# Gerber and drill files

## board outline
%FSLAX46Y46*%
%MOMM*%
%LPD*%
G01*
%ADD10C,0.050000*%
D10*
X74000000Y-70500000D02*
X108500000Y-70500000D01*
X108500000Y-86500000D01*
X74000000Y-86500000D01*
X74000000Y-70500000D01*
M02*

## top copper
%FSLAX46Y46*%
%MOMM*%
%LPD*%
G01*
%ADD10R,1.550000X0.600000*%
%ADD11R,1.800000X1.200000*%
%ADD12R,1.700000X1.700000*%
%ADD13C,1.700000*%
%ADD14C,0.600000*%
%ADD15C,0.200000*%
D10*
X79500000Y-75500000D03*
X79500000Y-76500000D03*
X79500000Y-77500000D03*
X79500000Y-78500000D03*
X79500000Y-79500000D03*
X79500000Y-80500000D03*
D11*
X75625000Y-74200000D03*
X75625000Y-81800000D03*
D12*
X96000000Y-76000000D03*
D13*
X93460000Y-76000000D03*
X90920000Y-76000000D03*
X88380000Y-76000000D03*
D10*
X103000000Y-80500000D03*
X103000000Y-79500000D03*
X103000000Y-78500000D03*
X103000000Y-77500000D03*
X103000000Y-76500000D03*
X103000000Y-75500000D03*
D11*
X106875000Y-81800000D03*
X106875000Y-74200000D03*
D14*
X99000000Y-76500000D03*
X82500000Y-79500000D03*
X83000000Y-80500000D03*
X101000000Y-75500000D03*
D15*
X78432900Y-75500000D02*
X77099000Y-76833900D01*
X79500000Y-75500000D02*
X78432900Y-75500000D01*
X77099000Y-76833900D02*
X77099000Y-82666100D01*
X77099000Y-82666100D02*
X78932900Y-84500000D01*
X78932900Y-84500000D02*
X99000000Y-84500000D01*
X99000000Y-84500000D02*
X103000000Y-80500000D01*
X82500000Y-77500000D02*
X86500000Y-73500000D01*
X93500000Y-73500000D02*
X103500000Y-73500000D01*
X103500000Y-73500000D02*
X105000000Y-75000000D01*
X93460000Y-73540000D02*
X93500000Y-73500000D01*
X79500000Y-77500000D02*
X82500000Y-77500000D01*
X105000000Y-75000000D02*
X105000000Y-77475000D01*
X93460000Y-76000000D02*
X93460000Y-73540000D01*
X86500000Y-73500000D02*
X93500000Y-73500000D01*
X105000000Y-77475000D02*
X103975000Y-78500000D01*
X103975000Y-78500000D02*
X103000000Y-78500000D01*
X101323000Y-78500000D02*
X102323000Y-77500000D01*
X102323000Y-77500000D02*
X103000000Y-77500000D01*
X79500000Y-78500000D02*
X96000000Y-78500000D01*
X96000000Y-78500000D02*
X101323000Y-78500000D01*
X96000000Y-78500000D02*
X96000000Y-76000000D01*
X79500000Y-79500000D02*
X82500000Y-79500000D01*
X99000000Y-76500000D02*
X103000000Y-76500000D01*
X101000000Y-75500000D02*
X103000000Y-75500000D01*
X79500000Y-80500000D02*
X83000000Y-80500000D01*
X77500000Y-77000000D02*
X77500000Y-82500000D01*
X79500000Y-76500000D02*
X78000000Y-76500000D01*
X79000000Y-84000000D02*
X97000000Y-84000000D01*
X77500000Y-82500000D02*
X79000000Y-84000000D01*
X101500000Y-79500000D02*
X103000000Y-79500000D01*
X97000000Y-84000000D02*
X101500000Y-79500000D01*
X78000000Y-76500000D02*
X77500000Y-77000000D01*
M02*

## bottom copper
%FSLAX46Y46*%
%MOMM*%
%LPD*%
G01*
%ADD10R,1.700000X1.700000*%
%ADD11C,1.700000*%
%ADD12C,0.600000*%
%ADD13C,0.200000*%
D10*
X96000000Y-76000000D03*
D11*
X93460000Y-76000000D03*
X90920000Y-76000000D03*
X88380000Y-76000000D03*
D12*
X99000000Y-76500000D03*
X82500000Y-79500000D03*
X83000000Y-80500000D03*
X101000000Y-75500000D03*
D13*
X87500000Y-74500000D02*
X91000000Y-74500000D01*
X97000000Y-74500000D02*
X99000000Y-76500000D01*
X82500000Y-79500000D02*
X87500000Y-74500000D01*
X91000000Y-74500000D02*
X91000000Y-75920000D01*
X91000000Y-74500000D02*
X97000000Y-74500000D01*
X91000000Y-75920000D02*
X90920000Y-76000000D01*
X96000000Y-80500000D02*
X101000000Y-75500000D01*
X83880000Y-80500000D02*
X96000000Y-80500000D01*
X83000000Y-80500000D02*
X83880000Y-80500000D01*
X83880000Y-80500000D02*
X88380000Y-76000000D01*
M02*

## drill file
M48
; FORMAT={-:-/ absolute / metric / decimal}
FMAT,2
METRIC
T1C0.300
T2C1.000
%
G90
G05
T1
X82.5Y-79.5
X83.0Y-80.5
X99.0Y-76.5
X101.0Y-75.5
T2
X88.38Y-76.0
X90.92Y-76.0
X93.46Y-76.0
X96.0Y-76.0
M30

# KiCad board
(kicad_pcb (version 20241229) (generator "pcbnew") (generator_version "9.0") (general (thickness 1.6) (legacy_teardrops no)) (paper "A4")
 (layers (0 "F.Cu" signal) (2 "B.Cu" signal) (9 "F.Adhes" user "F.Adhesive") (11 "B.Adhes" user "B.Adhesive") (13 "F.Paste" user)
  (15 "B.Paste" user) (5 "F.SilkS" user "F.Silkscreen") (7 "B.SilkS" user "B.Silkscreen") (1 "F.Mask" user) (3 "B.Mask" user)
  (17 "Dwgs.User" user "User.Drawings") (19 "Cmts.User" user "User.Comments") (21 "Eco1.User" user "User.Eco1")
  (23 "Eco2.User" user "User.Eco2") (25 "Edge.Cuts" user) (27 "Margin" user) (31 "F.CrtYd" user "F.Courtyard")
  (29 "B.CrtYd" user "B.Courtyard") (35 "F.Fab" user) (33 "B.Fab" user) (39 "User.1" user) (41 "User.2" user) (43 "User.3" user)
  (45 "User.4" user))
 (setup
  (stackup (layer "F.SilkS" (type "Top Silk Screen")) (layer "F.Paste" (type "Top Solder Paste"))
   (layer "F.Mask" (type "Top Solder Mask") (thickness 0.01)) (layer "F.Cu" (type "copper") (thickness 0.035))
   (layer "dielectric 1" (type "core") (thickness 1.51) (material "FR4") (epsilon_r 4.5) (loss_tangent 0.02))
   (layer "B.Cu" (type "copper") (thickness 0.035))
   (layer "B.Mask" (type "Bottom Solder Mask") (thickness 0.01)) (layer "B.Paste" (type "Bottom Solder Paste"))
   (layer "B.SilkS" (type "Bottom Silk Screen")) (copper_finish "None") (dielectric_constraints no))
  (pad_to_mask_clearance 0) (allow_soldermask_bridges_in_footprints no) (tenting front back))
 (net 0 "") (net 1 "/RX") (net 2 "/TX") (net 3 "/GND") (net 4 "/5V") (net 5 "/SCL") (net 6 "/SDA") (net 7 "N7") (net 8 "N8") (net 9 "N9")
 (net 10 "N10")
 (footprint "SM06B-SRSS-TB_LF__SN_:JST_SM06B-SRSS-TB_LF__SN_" (layer "F.Cu") (at 79.5 78 -90)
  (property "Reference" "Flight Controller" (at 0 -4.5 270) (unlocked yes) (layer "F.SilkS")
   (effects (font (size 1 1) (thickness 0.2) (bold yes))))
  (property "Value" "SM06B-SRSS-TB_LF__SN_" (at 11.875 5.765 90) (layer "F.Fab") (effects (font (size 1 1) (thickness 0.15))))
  (pad "1" smd rect (at -2.5 0 270) (size 0.6 1.55) (layers "F.Cu" "F.Mask" "F.Paste") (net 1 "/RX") (solder_mask_margin 0.102))
  (pad "2" smd rect (at -1.5 0 270) (size 0.6 1.55) (layers "F.Cu" "F.Mask" "F.Paste") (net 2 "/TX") (solder_mask_margin 0.102))
  (pad "3" smd rect (at -0.5 0 270) (size 0.6 1.55) (layers "F.Cu" "F.Mask" "F.Paste") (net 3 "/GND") (solder_mask_margin 0.102))
  (pad "4" smd rect (at 0.5 0 270) (size 0.6 1.55) (layers "F.Cu" "F.Mask" "F.Paste") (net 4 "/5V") (solder_mask_margin 0.102))
  (pad "5" smd rect (at 1.5 0 270) (size 0.6 1.55) (layers "F.Cu" "F.Mask" "F.Paste") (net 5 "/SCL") (solder_mask_margin 0.102))
  (pad "6" smd rect (at 2.5 0 270) (size 0.6 1.55) (layers "F.Cu" "F.Mask" "F.Paste") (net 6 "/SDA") (solder_mask_margin 0.102))
  (pad "S1" smd rect (at -3.8 3.875 270) (size 1.2 1.8) (layers "F.Cu" "F.Mask" "F.Paste") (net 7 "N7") (solder_mask_margin 0.102))
  (pad "S2" smd rect (at 3.8 3.875 270) (size 1.2 1.8) (layers "F.Cu" "F.Mask" "F.Paste") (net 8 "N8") (solder_mask_margin 0.102)))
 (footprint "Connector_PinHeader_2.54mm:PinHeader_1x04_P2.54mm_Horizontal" (layer "F.Cu") (at 96 76 -90)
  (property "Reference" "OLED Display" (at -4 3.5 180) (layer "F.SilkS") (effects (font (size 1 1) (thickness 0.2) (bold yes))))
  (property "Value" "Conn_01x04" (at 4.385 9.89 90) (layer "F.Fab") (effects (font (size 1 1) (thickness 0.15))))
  (pad "1" thru_hole rect (at 0 0 270) (size 1.7 1.7) (drill 1) (layers "*.Cu" "*.Mask") (remove_unused_layers no) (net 4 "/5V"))
  (pad "2" thru_hole circle (at 0 2.54 270) (size 1.7 1.7) (drill 1) (layers "*.Cu" "*.Mask") (remove_unused_layers no) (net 3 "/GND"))
  (pad "3" thru_hole circle (at 0 5.08 270) (size 1.7 1.7) (drill 1) (layers "*.Cu" "*.Mask") (remove_unused_layers no) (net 5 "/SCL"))
  (pad "4" thru_hole circle (at 0 7.62 270) (size 1.7 1.7) (drill 1) (layers "*.Cu" "*.Mask") (remove_unused_layers no) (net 6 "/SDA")))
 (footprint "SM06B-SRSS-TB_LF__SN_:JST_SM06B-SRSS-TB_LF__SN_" (layer "F.Cu") (at 103 78 90)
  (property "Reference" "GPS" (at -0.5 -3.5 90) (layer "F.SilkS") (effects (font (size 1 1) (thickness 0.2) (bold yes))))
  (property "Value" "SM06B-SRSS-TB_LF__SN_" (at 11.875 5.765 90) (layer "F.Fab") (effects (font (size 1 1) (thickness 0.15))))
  (pad "1" smd rect (at -2.5 0 90) (size 0.6 1.55) (layers "F.Cu" "F.Mask" "F.Paste") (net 1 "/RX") (solder_mask_margin 0.102))
  (pad "2" smd rect (at -1.5 0 90) (size 0.6 1.55) (layers "F.Cu" "F.Mask" "F.Paste") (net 2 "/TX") (solder_mask_margin 0.102))
  (pad "3" smd rect (at -0.5 0 90) (size 0.6 1.55) (layers "F.Cu" "F.Mask" "F.Paste") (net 3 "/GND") (solder_mask_margin 0.102))
  (pad "4" smd rect (at 0.5 0 90) (size 0.6 1.55) (layers "F.Cu" "F.Mask" "F.Paste") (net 4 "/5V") (solder_mask_margin 0.102))
  (pad "5" smd rect (at 1.5 0 90) (size 0.6 1.55) (layers "F.Cu" "F.Mask" "F.Paste") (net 5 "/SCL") (solder_mask_margin 0.102))
  (pad "6" smd rect (at 2.5 0 90) (size 0.6 1.55) (layers "F.Cu" "F.Mask" "F.Paste") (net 6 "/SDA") (solder_mask_margin 0.102))
  (pad "S1" smd rect (at -3.8 3.875 90) (size 1.2 1.8) (layers "F.Cu" "F.Mask" "F.Paste") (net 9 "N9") (solder_mask_margin 0.102))
  (pad "S2" smd rect (at 3.8 3.875 90) (size 1.2 1.8) (layers "F.Cu" "F.Mask" "F.Paste") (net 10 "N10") (solder_mask_margin 0.102)))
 (gr_rect (start 74 70.5) (end 108.5 86.5) (stroke (width 0.05) (type default)) (fill no) (layer "Edge.Cuts"))
 (segment (start 78.4329 75.5) (end 77.099 76.8339) (width 0.2) (layer "F.Cu") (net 1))
 (segment (start 79.5 75.5) (end 78.4329 75.5) (width 0.2) (layer "F.Cu") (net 1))
 (segment (start 77.099 76.8339) (end 77.099 82.6661) (width 0.2) (layer "F.Cu") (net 1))
 (segment (start 77.099 82.6661) (end 78.9329 84.5) (width 0.2) (layer "F.Cu") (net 1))
 (segment (start 78.9329 84.5) (end 99 84.5) (width 0.2) (layer "F.Cu") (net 1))
 (segment (start 99 84.5) (end 103 80.5) (width 0.2) (layer "F.Cu") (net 1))
 (segment (start 82.5 77.5) (end 86.5 73.5) (width 0.2) (layer "F.Cu") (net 3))
 (segment (start 93.5 73.5) (end 103.5 73.5) (width 0.2) (layer "F.Cu") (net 3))
 (segment (start 103.5 73.5) (end 105 75) (width 0.2) (layer "F.Cu") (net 3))
 (segment (start 93.46 73.54) (end 93.5 73.5) (width 0.2) (layer "F.Cu") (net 3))
 (segment (start 79.5 77.5) (end 82.5 77.5) (width 0.2) (layer "F.Cu") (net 3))
 (segment (start 105 75) (end 105 77.475) (width 0.2) (layer "F.Cu") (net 3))
 (segment (start 93.46 76) (end 93.46 73.54) (width 0.2) (layer "F.Cu") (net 3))
 (segment (start 86.5 73.5) (end 93.5 73.5) (width 0.2) (layer "F.Cu") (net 3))
 (segment (start 105 77.475) (end 103.975 78.5) (width 0.2) (layer "F.Cu") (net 3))
 (segment (start 103.975 78.5) (end 103 78.5) (width 0.2) (layer "F.Cu") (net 3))
 (segment (start 101.323 78.5) (end 102.323 77.5) (width 0.2) (layer "F.Cu") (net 4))
 (segment (start 102.323 77.5) (end 103 77.5) (width 0.2) (layer "F.Cu") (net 4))
 (segment (start 79.5 78.5) (end 96 78.5) (width 0.2) (layer "F.Cu") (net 4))
 (segment (start 96 78.5) (end 101.323 78.5) (width 0.2) (layer "F.Cu") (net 4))
 (segment (start 96 78.5) (end 96 76) (width 0.2) (layer "F.Cu") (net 4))
 (segment (start 79.5 79.5) (end 82.5 79.5) (width 0.2) (layer "F.Cu") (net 5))
 (segment (start 99 76.5) (end 103 76.5) (width 0.2) (layer "F.Cu") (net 5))
 (via (at 99 76.5) (size 0.6) (drill 0.3) (layers "F.Cu" "B.Cu") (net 5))
 (via (at 82.5 79.5) (size 0.6) (drill 0.3) (layers "F.Cu" "B.Cu") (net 5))
 (segment (start 87.5 74.5) (end 91 74.5) (width 0.2) (layer "B.Cu") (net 5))
 (segment (start 97 74.5) (end 99 76.5) (width 0.2) (layer "B.Cu") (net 5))
 (segment (start 82.5 79.5) (end 87.5 74.5) (width 0.2) (layer "B.Cu") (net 5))
 (segment (start 91 74.5) (end 91 75.92) (width 0.2) (layer "B.Cu") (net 5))
 (segment (start 91 74.5) (end 97 74.5) (width 0.2) (layer "B.Cu") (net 5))
 (segment (start 91 75.92) (end 90.92 76) (width 0.2) (layer "B.Cu") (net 5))
 (segment (start 101 75.5) (end 103 75.5) (width 0.2) (layer "F.Cu") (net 6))
 (segment (start 79.5 80.5) (end 83 80.5) (width 0.2) (layer "F.Cu") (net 6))
 (via (at 83 80.5) (size 0.6) (drill 0.3) (layers "F.Cu" "B.Cu") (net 6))
 (via (at 101 75.5) (size 0.6) (drill 0.3) (layers "F.Cu" "B.Cu") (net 6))
 (segment (start 96 80.5) (end 101 75.5) (width 0.2) (layer "B.Cu") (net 6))
 (segment (start 83.88 80.5) (end 96 80.5) (width 0.2) (layer "B.Cu") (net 6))
 (segment (start 83 80.5) (end 83.88 80.5) (width 0.2) (layer "B.Cu") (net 6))
 (segment (start 83.88 80.5) (end 88.38 76) (width 0.2) (layer "B.Cu") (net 6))
 (segment (start 77.5 77) (end 77.5 82.5) (width 0.2) (layer "F.Cu") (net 2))
 (segment (start 79.5 76.5) (end 78 76.5) (width 0.2) (layer "F.Cu") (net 2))
 (segment (start 79 84) (end 97 84) (width 0.2) (layer "F.Cu") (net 2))
 (segment (start 77.5 82.5) (end 79 84) (width 0.2) (layer "F.Cu") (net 2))
 (segment (start 101.5 79.5) (end 103 79.5) (width 0.2) (layer "F.Cu") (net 2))
 (segment (start 97 84) (end 101.5 79.5) (width 0.2) (layer "F.Cu") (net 2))
 (segment (start 78 76.5) (end 77.5 77) (width 0.2) (layer "F.Cu") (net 2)))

